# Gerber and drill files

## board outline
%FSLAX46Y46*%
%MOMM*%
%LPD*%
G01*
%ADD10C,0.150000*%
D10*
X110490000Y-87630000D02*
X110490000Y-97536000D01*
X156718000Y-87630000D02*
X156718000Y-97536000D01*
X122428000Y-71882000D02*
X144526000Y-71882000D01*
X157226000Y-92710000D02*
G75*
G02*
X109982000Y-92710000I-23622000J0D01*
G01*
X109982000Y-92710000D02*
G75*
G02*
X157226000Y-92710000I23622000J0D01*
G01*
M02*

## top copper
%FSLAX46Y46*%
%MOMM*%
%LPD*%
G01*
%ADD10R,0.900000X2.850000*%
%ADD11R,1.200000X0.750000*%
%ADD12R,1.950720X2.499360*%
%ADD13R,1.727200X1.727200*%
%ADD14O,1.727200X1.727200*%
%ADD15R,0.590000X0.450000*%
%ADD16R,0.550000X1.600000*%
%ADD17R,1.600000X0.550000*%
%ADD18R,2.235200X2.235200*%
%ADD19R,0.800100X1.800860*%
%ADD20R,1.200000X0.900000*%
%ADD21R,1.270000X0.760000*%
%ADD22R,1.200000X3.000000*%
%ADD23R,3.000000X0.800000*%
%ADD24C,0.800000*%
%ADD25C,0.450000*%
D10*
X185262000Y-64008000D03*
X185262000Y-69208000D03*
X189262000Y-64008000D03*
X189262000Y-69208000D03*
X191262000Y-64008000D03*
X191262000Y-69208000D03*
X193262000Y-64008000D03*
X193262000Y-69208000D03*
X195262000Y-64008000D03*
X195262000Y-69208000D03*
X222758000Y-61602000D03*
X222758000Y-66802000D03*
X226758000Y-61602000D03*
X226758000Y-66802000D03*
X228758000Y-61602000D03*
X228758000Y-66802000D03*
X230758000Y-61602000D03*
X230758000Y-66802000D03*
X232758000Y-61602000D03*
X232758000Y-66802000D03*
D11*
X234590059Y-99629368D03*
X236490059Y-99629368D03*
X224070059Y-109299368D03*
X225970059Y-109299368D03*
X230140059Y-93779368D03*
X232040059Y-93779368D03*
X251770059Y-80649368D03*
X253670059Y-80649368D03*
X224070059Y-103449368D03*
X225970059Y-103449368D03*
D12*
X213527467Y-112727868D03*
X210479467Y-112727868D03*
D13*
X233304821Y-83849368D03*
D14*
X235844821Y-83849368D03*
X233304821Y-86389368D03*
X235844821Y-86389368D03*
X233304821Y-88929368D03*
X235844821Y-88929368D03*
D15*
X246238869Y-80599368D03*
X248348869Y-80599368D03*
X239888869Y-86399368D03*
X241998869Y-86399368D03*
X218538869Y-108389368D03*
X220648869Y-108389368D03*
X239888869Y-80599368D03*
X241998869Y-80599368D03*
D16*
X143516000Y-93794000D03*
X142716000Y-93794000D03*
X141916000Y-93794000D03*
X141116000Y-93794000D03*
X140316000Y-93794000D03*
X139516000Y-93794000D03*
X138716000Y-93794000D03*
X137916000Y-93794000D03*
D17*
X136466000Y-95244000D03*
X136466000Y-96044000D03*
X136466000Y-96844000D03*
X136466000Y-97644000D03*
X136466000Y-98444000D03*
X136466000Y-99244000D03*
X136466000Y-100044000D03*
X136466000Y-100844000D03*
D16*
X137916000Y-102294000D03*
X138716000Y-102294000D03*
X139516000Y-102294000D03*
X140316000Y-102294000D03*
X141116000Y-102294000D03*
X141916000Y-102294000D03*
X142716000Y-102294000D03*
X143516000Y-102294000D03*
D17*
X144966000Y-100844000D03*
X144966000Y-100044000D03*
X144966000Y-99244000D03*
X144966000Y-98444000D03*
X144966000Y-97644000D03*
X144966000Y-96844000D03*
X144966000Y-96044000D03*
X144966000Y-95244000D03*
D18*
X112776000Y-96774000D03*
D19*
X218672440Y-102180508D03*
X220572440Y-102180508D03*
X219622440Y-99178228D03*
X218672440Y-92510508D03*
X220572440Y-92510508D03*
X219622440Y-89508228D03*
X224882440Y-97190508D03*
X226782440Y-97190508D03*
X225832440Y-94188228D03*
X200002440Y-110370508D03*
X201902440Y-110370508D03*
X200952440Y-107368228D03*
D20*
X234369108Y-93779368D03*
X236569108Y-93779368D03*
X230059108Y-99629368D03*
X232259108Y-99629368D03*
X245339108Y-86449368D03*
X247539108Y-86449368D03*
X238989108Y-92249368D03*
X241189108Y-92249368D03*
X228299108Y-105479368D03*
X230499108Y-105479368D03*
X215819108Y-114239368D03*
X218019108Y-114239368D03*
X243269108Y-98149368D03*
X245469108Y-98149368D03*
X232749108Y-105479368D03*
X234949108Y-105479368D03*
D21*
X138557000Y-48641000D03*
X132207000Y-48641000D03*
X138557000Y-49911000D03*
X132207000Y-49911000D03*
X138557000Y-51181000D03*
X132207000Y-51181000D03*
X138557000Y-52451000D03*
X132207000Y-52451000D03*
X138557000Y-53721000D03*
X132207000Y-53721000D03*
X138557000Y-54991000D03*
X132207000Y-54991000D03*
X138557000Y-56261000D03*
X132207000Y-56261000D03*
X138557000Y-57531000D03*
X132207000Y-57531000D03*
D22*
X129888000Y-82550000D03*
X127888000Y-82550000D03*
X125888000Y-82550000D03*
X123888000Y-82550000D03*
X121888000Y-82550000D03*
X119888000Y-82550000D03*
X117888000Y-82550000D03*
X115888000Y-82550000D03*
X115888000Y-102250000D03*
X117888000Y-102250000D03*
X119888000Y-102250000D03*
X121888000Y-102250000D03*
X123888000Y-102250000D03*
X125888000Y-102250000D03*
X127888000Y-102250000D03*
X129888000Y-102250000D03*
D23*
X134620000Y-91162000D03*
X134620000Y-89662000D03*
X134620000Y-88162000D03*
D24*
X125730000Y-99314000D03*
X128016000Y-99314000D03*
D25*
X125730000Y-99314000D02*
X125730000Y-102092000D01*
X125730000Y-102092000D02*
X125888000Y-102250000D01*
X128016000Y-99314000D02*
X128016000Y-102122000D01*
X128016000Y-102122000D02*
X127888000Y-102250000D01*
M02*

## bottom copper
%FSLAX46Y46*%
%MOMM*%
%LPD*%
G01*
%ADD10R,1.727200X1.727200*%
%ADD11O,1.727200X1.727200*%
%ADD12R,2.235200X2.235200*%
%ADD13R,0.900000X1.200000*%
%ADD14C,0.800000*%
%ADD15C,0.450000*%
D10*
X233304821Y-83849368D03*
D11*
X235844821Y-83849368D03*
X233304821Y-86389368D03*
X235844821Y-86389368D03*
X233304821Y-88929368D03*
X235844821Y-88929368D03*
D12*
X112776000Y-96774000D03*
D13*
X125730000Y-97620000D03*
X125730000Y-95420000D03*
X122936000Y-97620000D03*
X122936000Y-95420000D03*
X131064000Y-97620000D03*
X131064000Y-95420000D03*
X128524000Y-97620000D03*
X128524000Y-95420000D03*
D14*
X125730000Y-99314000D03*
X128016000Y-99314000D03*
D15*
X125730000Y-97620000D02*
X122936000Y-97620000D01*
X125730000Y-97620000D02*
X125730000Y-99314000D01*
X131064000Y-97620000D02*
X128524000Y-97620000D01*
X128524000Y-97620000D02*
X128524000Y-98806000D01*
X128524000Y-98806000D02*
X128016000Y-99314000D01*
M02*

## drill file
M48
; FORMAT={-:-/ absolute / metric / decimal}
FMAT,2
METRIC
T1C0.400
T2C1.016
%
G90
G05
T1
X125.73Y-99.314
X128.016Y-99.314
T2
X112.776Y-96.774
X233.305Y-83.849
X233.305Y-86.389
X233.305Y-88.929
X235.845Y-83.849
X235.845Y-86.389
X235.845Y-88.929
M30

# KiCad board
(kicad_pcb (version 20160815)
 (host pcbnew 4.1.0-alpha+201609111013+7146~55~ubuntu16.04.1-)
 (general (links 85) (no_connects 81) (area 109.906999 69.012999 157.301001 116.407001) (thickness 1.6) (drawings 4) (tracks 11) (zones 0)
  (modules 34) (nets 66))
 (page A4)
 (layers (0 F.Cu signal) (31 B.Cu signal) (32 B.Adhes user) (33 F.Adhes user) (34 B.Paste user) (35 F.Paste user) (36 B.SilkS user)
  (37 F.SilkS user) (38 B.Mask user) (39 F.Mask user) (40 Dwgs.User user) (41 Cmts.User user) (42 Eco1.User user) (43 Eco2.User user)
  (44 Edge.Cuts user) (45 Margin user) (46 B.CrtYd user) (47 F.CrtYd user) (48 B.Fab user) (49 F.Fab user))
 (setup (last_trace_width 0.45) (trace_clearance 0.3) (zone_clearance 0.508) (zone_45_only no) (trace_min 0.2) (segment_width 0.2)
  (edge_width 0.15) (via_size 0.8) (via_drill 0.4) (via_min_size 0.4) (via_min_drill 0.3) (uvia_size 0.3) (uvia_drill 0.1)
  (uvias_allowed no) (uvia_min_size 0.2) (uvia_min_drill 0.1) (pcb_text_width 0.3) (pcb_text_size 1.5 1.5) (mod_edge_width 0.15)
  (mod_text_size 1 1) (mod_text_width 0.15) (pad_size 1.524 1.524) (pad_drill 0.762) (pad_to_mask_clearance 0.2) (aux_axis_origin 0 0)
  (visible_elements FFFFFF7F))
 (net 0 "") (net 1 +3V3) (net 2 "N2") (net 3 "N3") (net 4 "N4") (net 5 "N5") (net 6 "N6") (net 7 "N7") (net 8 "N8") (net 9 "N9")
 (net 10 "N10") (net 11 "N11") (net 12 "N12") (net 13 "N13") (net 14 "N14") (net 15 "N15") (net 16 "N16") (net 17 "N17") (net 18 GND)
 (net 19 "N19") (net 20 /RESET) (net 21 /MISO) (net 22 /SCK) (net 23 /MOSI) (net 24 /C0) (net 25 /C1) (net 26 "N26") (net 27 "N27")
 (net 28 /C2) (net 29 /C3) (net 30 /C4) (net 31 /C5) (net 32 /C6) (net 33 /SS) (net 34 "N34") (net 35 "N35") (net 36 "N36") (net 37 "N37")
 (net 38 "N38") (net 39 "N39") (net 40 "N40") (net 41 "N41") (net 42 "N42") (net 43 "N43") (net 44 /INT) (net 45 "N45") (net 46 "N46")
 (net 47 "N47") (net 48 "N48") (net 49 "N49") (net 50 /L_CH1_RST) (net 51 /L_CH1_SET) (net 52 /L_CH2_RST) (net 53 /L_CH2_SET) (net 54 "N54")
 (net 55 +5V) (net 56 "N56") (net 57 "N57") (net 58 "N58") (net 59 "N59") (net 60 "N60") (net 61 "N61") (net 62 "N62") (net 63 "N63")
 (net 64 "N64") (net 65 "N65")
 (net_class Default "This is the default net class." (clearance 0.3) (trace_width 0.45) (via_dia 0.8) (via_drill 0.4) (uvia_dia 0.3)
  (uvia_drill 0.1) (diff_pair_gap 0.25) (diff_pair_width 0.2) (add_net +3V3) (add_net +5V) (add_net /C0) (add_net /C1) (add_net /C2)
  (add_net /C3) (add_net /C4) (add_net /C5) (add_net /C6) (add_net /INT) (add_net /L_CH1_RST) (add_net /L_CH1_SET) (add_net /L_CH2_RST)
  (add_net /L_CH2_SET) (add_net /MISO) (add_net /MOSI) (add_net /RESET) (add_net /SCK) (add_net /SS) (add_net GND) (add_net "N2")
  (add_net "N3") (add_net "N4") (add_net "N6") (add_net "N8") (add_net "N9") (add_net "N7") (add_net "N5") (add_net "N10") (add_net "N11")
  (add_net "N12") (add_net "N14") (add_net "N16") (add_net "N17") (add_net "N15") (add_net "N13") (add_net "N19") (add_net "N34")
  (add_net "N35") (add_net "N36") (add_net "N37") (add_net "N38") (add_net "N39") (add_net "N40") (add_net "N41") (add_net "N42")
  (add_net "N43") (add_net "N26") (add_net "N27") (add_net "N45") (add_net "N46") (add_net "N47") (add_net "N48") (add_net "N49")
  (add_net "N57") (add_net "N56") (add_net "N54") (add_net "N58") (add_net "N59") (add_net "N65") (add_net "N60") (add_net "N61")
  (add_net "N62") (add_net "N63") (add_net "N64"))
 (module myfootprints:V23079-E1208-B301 (layer F.Cu) (at 190.262 66.608)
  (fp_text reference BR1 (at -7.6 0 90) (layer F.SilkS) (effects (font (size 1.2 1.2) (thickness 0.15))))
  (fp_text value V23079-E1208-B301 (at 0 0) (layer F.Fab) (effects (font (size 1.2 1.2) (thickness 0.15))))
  (pad 12 smd rect (at -5 -2.6) (size 0.9 2.85) (layers F.Cu F.Paste F.Mask) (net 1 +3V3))
  (pad 1 smd rect (at -5 2.6) (size 0.9 2.85) (layers F.Cu F.Paste F.Mask) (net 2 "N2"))
  (pad 10 smd rect (at -1 -2.6) (size 0.9 2.85) (layers F.Cu F.Paste F.Mask) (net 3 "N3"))
  (pad 3 smd rect (at -1 2.6) (size 0.9 2.85) (layers F.Cu F.Paste F.Mask) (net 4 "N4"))
  (pad 9 smd rect (at 1 -2.6) (size 0.9 2.85) (layers F.Cu F.Paste F.Mask) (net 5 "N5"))
  (pad 4 smd rect (at 1 2.6) (size 0.9 2.85) (layers F.Cu F.Paste F.Mask) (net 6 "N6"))
  (pad 8 smd rect (at 3 -2.6) (size 0.9 2.85) (layers F.Cu F.Paste F.Mask) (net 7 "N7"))
  (pad 5 smd rect (at 3 2.6) (size 0.9 2.85) (layers F.Cu F.Paste F.Mask) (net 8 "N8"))
  (pad 7 smd rect (at 5 -2.6) (size 0.9 2.85) (layers F.Cu F.Paste F.Mask) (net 1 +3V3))
  (pad 6 smd rect (at 5 2.6) (size 0.9 2.85) (layers F.Cu F.Paste F.Mask) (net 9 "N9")))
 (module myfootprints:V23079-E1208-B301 (layer F.Cu) (at 227.758 64.202)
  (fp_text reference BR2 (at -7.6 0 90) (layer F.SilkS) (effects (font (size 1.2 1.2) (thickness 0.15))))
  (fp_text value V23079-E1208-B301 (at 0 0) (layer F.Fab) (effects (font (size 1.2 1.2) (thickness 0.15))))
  (pad 12 smd rect (at -5 -2.6) (size 0.9 2.85) (layers F.Cu F.Paste F.Mask) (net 1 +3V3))
  (pad 1 smd rect (at -5 2.6) (size 0.9 2.85) (layers F.Cu F.Paste F.Mask) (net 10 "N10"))
  (pad 10 smd rect (at -1 -2.6) (size 0.9 2.85) (layers F.Cu F.Paste F.Mask) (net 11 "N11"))
  (pad 3 smd rect (at -1 2.6) (size 0.9 2.85) (layers F.Cu F.Paste F.Mask) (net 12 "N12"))
  (pad 9 smd rect (at 1 -2.6) (size 0.9 2.85) (layers F.Cu F.Paste F.Mask) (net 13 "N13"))
  (pad 4 smd rect (at 1 2.6) (size 0.9 2.85) (layers F.Cu F.Paste F.Mask) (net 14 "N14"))
  (pad 8 smd rect (at 3 -2.6) (size 0.9 2.85) (layers F.Cu F.Paste F.Mask) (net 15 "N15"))
  (pad 5 smd rect (at 3 2.6) (size 0.9 2.85) (layers F.Cu F.Paste F.Mask) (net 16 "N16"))
  (pad 7 smd rect (at 5 -2.6) (size 0.9 2.85) (layers F.Cu F.Paste F.Mask) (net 1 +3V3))
  (pad 6 smd rect (at 5 2.6) (size 0.9 2.85) (layers F.Cu F.Paste F.Mask) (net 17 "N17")))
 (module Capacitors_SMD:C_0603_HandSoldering (layer F.Cu) (at 235.540059 99.629368)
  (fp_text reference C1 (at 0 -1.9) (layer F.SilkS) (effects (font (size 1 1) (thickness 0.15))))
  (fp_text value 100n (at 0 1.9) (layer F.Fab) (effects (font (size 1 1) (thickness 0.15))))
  (pad 1 smd rect (at -0.95 0) (size 1.2 0.75) (layers F.Cu F.Paste F.Mask) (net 1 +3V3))
  (pad 2 smd rect (at 0.95 0) (size 1.2 0.75) (layers F.Cu F.Paste F.Mask) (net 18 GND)))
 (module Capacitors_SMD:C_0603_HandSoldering (layer F.Cu) (at 225.020059 109.299368)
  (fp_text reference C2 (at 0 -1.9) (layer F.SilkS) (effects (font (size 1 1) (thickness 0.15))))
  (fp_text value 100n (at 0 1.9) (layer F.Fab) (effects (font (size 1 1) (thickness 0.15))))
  (pad 1 smd rect (at -0.95 0) (size 1.2 0.75) (layers F.Cu F.Paste F.Mask) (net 18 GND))
  (pad 2 smd rect (at 0.95 0) (size 1.2 0.75) (layers F.Cu F.Paste F.Mask) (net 1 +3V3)))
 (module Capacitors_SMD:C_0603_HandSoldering (layer F.Cu) (at 231.090059 93.779368)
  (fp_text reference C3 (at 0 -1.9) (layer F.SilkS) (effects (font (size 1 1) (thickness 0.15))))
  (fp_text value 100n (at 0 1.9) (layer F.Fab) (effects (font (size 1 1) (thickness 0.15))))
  (pad 1 smd rect (at -0.95 0) (size 1.2 0.75) (layers F.Cu F.Paste F.Mask) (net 18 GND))
  (pad 2 smd rect (at 0.95 0) (size 1.2 0.75) (layers F.Cu F.Paste F.Mask) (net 1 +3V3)))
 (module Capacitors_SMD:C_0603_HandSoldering (layer F.Cu) (at 252.720059 80.649368)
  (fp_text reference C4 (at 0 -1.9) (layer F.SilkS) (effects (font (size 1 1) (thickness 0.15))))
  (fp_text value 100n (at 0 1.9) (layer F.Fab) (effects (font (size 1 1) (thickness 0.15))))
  (pad 1 smd rect (at -0.95 0) (size 1.2 0.75) (layers F.Cu F.Paste F.Mask) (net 18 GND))
  (pad 2 smd rect (at 0.95 0) (size 1.2 0.75) (layers F.Cu F.Paste F.Mask) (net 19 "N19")))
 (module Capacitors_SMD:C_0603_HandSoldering (layer F.Cu) (at 225.020059 103.449368)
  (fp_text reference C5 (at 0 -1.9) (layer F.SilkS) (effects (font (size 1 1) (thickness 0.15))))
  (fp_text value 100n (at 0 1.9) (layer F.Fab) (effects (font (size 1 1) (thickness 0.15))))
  (pad 1 smd rect (at -0.95 0) (size 1.2 0.75) (layers F.Cu F.Paste F.Mask) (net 18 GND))
  (pad 2 smd rect (at 0.95 0) (size 1.2 0.75) (layers F.Cu F.Paste F.Mask) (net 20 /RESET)))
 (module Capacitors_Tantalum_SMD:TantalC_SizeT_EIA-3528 (layer F.Cu) (at 212.003467 112.727868)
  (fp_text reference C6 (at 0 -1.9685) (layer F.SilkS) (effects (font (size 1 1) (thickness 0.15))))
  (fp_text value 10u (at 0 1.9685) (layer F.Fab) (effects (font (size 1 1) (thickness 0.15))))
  (pad 1 smd rect (at 1.524 0) (size 1.95072 2.49936) (layers F.Cu F.Paste F.Mask) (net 1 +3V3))
  (pad 2 smd rect (at -1.524 0) (size 1.95072 2.49936) (layers F.Cu F.Paste F.Mask) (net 18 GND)))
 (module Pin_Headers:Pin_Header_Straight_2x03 (layer F.Cu) (at 233.304821 83.849368)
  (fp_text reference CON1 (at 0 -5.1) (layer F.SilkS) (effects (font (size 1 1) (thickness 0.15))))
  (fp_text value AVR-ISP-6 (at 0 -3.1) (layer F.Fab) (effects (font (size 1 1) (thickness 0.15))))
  (pad 1 thru_hole rect (at 0 0) (size 1.7272 1.7272) (drill 1.016) (layers *.Cu *.Mask F.SilkS) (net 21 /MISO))
  (pad 2 thru_hole oval (at 2.54 0) (size 1.7272 1.7272) (drill 1.016) (layers *.Cu *.Mask F.SilkS) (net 1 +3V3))
  (pad 3 thru_hole oval (at 0 2.54) (size 1.7272 1.7272) (drill 1.016) (layers *.Cu *.Mask F.SilkS) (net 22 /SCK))
  (pad 4 thru_hole oval (at 2.54 2.54) (size 1.7272 1.7272) (drill 1.016) (layers *.Cu *.Mask F.SilkS) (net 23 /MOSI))
  (pad 5 thru_hole oval (at 0 5.08) (size 1.7272 1.7272) (drill 1.016) (layers *.Cu *.Mask F.SilkS) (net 20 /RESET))
  (pad 6 thru_hole oval (at 2.54 5.08) (size 1.7272 1.7272) (drill 1.016) (layers *.Cu *.Mask F.SilkS) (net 18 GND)))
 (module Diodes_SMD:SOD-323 (layer F.Cu) (at 247.293869 80.599368)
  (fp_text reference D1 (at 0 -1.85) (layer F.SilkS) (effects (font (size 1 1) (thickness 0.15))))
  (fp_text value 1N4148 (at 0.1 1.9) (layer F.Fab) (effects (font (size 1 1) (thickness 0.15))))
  (pad 1 smd rect (at -1.055 0) (size 0.59 0.45) (layers F.Cu F.Paste F.Mask) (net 1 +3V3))
  (pad 2 smd rect (at 1.055 0) (size 0.59 0.45) (layers F.Cu F.Paste F.Mask) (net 2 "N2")))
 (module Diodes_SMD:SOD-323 (layer F.Cu) (at 240.943869 86.399368)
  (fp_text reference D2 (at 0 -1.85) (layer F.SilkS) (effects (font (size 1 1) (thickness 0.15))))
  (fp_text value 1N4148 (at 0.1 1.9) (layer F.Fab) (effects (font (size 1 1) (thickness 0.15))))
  (pad 1 smd rect (at -1.055 0) (size 0.59 0.45) (layers F.Cu F.Paste F.Mask) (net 1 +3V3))
  (pad 2 smd rect (at 1.055 0) (size 0.59 0.45) (layers F.Cu F.Paste F.Mask) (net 9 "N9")))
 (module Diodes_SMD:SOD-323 (layer F.Cu) (at 219.593869 108.389368)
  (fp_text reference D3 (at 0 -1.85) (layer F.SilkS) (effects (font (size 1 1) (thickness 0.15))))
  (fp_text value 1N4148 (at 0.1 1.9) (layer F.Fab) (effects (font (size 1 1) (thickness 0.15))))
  (pad 1 smd rect (at -1.055 0) (size 0.59 0.45) (layers F.Cu F.Paste F.Mask) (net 1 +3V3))
  (pad 2 smd rect (at 1.055 0) (size 0.59 0.45) (layers F.Cu F.Paste F.Mask) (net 10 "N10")))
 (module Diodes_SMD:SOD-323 (layer F.Cu) (at 240.943869 80.599368)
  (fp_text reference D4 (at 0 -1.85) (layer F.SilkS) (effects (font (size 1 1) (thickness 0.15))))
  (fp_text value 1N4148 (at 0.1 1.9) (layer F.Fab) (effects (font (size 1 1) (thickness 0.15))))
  (pad 1 smd rect (at -1.055 0) (size 0.59 0.45) (layers F.Cu F.Paste F.Mask) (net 1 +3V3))
  (pad 2 smd rect (at 1.055 0) (size 0.59 0.45) (layers F.Cu F.Paste F.Mask) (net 17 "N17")))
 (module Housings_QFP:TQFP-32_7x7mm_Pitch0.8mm (layer F.Cu) (at 140.716 98.044 270)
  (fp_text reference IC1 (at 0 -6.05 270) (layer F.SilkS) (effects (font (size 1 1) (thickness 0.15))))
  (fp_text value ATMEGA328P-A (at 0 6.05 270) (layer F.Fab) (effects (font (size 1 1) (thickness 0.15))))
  (pad 1 smd rect (at -4.25 -2.8 270) (size 1.6 0.55) (layers F.Cu F.Paste F.Mask) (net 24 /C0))
  (pad 2 smd rect (at -4.25 -2 270) (size 1.6 0.55) (layers F.Cu F.Paste F.Mask) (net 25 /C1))
  (pad 3 smd rect (at -4.25 -1.2 270) (size 1.6 0.55) (layers F.Cu F.Paste F.Mask) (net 18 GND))
  (pad 4 smd rect (at -4.25 -0.4 270) (size 1.6 0.55) (layers F.Cu F.Paste F.Mask) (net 1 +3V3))
  (pad 5 smd rect (at -4.25 0.4 270) (size 1.6 0.55) (layers F.Cu F.Paste F.Mask) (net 18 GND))
  (pad 6 smd rect (at -4.25 1.2 270) (size 1.6 0.55) (layers F.Cu F.Paste F.Mask) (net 1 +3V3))
  (pad 7 smd rect (at -4.25 2 270) (size 1.6 0.55) (layers F.Cu F.Paste F.Mask) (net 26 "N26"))
  (pad 8 smd rect (at -4.25 2.8 270) (size 1.6 0.55) (layers F.Cu F.Paste F.Mask) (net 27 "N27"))
  (pad 9 smd rect (at -2.8 4.25) (size 1.6 0.55) (layers F.Cu F.Paste F.Mask) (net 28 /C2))
  (pad 10 smd rect (at -2 4.25) (size 1.6 0.55) (layers F.Cu F.Paste F.Mask) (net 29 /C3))
  (pad 11 smd rect (at -1.2 4.25) (size 1.6 0.55) (layers F.Cu F.Paste F.Mask) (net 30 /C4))
  (pad 12 smd rect (at -0.4 4.25) (size 1.6 0.55) (layers F.Cu F.Paste F.Mask) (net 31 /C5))
  (pad 13 smd rect (at 0.4 4.25) (size 1.6 0.55) (layers F.Cu F.Paste F.Mask) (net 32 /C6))
  (pad 14 smd rect (at 1.2 4.25) (size 1.6 0.55) (layers F.Cu F.Paste F.Mask) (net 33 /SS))
  (pad 15 smd rect (at 2 4.25) (size 1.6 0.55) (layers F.Cu F.Paste F.Mask) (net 23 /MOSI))
  (pad 16 smd rect (at 2.8 4.25) (size 1.6 0.55) (layers F.Cu F.Paste F.Mask) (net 21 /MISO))
  (pad 17 smd rect (at 4.25 2.8 270) (size 1.6 0.55) (layers F.Cu F.Paste F.Mask) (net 22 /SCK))
  (pad 18 smd rect (at 4.25 2 270) (size 1.6 0.55) (layers F.Cu F.Paste F.Mask) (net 1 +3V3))
  (pad 19 smd rect (at 4.25 1.2 270) (size 1.6 0.55) (layers F.Cu F.Paste F.Mask) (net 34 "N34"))
  (pad 20 smd rect (at 4.25 0.4 270) (size 1.6 0.55) (layers F.Cu F.Paste F.Mask) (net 19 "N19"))
  (pad 21 smd rect (at 4.25 -0.4 270) (size 1.6 0.55) (layers F.Cu F.Paste F.Mask) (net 18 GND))
  (pad 22 smd rect (at 4.25 -1.2 270) (size 1.6 0.55) (layers F.Cu F.Paste F.Mask) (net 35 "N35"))
  (pad 23 smd rect (at 4.25 -2 270) (size 1.6 0.55) (layers F.Cu F.Paste F.Mask) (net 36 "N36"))
  (pad 24 smd rect (at 4.25 -2.8 270) (size 1.6 0.55) (layers F.Cu F.Paste F.Mask) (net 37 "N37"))
  (pad 25 smd rect (at 2.8 -4.25) (size 1.6 0.55) (layers F.Cu F.Paste F.Mask) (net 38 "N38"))
  (pad 26 smd rect (at 2 -4.25) (size 1.6 0.55) (layers F.Cu F.Paste F.Mask) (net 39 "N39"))
  (pad 27 smd rect (at 1.2 -4.25) (size 1.6 0.55) (layers F.Cu F.Paste F.Mask) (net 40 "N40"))
  (pad 28 smd rect (at 0.4 -4.25) (size 1.6 0.55) (layers F.Cu F.Paste F.Mask) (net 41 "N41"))
  (pad 29 smd rect (at -0.4 -4.25) (size 1.6 0.55) (layers F.Cu F.Paste F.Mask) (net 20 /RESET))
  (pad 30 smd rect (at -1.2 -4.25) (size 1.6 0.55) (layers F.Cu F.Paste F.Mask) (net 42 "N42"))
  (pad 31 smd rect (at -2 -4.25) (size 1.6 0.55) (layers F.Cu F.Paste F.Mask) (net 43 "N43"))
  (pad 32 smd rect (at -2.8 -4.25) (size 1.6 0.55) (layers F.Cu F.Paste F.Mask) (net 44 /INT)))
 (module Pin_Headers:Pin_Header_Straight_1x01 (layer F.Cu) (at 112.776 96.774)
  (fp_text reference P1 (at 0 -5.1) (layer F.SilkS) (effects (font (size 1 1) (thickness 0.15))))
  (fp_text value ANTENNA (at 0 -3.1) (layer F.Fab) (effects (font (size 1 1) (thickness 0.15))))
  (pad 1 thru_hole rect (at 0 0) (size 2.2352 2.2352) (drill 1.016) (layers *.Cu *.Mask F.SilkS) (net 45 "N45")))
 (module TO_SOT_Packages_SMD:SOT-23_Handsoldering (layer F.Cu) (at 219.62244 100.679368)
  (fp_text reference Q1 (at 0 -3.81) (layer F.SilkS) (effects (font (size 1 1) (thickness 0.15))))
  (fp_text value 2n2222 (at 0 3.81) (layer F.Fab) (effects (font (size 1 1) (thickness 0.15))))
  (pad 1 smd rect (at -0.95 1.50114) (size 0.8001 1.80086) (layers F.Cu F.Paste F.Mask) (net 2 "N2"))
  (pad 2 smd rect (at 0.95 1.50114) (size 0.8001 1.80086) (layers F.Cu F.Paste F.Mask) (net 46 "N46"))
  (pad 3 smd rect (at 0 -1.50114) (size 0.8001 1.80086) (layers F.Cu F.Paste F.Mask) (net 18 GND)))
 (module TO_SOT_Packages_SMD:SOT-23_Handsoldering (layer F.Cu) (at 219.62244 91.009368)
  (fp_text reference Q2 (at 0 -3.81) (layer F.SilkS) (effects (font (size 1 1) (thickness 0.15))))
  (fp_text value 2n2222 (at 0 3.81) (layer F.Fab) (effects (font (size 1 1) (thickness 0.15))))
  (pad 1 smd rect (at -0.95 1.50114) (size 0.8001 1.80086) (layers F.Cu F.Paste F.Mask) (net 9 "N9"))
  (pad 2 smd rect (at 0.95 1.50114) (size 0.8001 1.80086) (layers F.Cu F.Paste F.Mask) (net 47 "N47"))
  (pad 3 smd rect (at 0 -1.50114) (size 0.8001 1.80086) (layers F.Cu F.Paste F.Mask) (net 18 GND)))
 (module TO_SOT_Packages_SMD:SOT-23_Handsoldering (layer F.Cu) (at 225.83244 95.689368)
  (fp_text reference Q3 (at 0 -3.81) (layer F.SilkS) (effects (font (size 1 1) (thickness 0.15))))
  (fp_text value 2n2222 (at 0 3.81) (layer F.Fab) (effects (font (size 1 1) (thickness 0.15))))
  (pad 1 smd rect (at -0.95 1.50114) (size 0.8001 1.80086) (layers F.Cu F.Paste F.Mask) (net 10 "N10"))
  (pad 2 smd rect (at 0.95 1.50114) (size 0.8001 1.80086) (layers F.Cu F.Paste F.Mask) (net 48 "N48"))
  (pad 3 smd rect (at 0 -1.50114) (size 0.8001 1.80086) (layers F.Cu F.Paste F.Mask) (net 18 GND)))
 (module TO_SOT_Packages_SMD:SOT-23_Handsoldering (layer F.Cu) (at 200.95244 108.869368)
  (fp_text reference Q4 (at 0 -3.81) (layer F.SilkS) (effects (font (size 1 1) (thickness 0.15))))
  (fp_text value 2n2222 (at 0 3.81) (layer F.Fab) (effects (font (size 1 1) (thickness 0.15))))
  (pad 1 smd rect (at -0.95 1.50114) (size 0.8001 1.80086) (layers F.Cu F.Paste F.Mask) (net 17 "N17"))
  (pad 2 smd rect (at 0.95 1.50114) (size 0.8001 1.80086) (layers F.Cu F.Paste F.Mask) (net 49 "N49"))
  (pad 3 smd rect (at 0 -1.50114) (size 0.8001 1.80086) (layers F.Cu F.Paste F.Mask) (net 18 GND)))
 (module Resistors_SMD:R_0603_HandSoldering (layer F.Cu) (at 235.469108 93.779368)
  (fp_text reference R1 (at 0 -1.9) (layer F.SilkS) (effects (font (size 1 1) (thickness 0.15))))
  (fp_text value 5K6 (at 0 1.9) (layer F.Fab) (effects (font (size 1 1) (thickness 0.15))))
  (pad 1 smd rect (at -1.1 0) (size 1.2 0.9) (layers F.Cu F.Paste F.Mask) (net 46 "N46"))
  (pad 2 smd rect (at 1.1 0) (size 1.2 0.9) (layers F.Cu F.Paste F.Mask) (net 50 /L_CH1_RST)))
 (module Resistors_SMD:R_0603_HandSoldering (layer F.Cu) (at 231.159108 99.629368)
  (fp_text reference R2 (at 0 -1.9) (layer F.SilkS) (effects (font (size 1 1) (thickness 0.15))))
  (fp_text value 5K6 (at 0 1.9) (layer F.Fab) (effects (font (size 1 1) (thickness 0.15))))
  (pad 1 smd rect (at -1.1 0) (size 1.2 0.9) (layers F.Cu F.Paste F.Mask) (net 47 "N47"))
  (pad 2 smd rect (at 1.1 0) (size 1.2 0.9) (layers F.Cu F.Paste F.Mask) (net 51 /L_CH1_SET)))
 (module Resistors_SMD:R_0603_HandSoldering (layer F.Cu) (at 246.439108 86.449368)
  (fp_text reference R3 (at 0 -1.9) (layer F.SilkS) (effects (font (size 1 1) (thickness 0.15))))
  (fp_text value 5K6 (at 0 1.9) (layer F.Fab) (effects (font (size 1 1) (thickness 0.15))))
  (pad 1 smd rect (at -1.1 0) (size 1.2 0.9) (layers F.Cu F.Paste F.Mask) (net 48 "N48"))
  (pad 2 smd rect (at 1.1 0) (size 1.2 0.9) (layers F.Cu F.Paste F.Mask) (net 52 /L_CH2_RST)))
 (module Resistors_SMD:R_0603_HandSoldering (layer F.Cu) (at 240.089108 92.249368)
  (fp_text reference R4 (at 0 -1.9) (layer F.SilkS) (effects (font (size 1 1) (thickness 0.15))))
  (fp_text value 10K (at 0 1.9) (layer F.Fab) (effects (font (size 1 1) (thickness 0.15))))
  (pad 1 smd rect (at -1.1 0) (size 1.2 0.9) (layers F.Cu F.Paste F.Mask) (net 1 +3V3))
  (pad 2 smd rect (at 1.1 0) (size 1.2 0.9) (layers F.Cu F.Paste F.Mask) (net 20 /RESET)))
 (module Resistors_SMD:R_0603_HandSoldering (layer F.Cu) (at 229.399108 105.479368)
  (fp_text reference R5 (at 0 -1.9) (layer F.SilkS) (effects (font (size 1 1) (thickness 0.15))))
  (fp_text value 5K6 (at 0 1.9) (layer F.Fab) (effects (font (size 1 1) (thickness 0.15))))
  (pad 1 smd rect (at -1.1 0) (size 1.2 0.9) (layers F.Cu F.Paste F.Mask) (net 49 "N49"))
  (pad 2 smd rect (at 1.1 0) (size 1.2 0.9) (layers F.Cu F.Paste F.Mask) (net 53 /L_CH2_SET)))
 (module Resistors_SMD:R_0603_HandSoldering (layer B.Cu) (at 125.73 96.52 90)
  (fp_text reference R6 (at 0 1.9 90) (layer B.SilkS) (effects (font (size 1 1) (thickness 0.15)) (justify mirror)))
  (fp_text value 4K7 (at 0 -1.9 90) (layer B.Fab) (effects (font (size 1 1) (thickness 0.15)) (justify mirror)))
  (pad 1 smd rect (at -1.1 0 90) (size 1.2 0.9) (layers B.Cu B.Paste B.Mask) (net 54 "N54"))
  (pad 2 smd rect (at 1.1 0 90) (size 1.2 0.9) (layers B.Cu B.Paste B.Mask) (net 23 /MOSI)))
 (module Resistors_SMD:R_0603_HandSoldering (layer B.Cu) (at 122.936 96.52 90)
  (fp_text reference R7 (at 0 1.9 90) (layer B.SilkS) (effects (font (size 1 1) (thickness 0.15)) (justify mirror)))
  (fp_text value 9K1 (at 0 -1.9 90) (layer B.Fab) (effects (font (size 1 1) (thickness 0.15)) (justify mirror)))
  (pad 1 smd rect (at -1.1 0 90) (size 1.2 0.9) (layers B.Cu B.Paste B.Mask) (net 54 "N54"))
  (pad 2 smd rect (at 1.1 0 90) (size 1.2 0.9) (layers B.Cu B.Paste B.Mask) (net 18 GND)))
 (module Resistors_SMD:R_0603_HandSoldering (layer F.Cu) (at 216.919108 114.239368)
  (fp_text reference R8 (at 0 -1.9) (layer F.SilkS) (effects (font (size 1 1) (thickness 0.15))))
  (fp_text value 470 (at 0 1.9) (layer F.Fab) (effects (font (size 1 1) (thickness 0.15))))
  (pad 1 smd rect (at -1.1 0) (size 1.2 0.9) (layers F.Cu F.Paste F.Mask) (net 33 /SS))
  (pad 2 smd rect (at 1.1 0) (size 1.2 0.9) (layers F.Cu F.Paste F.Mask) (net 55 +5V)))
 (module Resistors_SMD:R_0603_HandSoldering (layer B.Cu) (at 131.064 96.52 90)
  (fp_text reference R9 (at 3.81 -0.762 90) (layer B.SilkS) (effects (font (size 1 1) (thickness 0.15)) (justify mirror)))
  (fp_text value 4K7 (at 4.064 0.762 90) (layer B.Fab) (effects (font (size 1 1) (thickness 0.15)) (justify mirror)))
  (pad 1 smd rect (at -1.1 0 90) (size 1.2 0.9) (layers B.Cu B.Paste B.Mask) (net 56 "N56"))
  (pad 2 smd rect (at 1.1 0 90) (size 1.2 0.9) (layers B.Cu B.Paste B.Mask) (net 33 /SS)))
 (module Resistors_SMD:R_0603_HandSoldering (layer F.Cu) (at 244.369108 98.149368)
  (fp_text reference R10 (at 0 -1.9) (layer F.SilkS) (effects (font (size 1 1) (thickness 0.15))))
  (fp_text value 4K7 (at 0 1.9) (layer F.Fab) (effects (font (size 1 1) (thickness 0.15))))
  (pad 1 smd rect (at -1.1 0) (size 1.2 0.9) (layers F.Cu F.Paste F.Mask) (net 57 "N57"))
  (pad 2 smd rect (at 1.1 0) (size 1.2 0.9) (layers F.Cu F.Paste F.Mask) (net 22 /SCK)))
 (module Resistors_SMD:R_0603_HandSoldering (layer B.Cu) (at 128.524 96.52 90)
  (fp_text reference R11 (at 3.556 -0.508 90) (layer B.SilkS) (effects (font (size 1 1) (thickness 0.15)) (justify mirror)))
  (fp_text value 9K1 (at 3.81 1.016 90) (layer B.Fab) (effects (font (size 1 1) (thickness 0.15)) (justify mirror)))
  (pad 1 smd rect (at -1.1 0 90) (size 1.2 0.9) (layers B.Cu B.Paste B.Mask) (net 56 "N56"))
  (pad 2 smd rect (at 1.1 0 90) (size 1.2 0.9) (layers B.Cu B.Paste B.Mask) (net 18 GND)))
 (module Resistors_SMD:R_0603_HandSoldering (layer F.Cu) (at 233.849108 105.479368)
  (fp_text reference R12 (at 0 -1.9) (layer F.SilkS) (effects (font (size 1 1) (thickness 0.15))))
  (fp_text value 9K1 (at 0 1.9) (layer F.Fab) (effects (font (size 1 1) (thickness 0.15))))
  (pad 1 smd rect (at -1.1 0) (size 1.2 0.9) (layers F.Cu F.Paste F.Mask) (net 57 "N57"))
  (pad 2 smd rect (at 1.1 0) (size 1.2 0.9) (layers F.Cu F.Paste F.Mask) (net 18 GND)))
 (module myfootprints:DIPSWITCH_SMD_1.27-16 (layer F.Cu) (at 135.382 53.086 270)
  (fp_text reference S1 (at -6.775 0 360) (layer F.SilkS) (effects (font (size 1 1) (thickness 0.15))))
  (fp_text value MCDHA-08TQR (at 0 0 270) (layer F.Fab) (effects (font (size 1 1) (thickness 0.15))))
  (pad 16 smd rect (at -4.445 -3.175 270) (size 0.76 1.27) (layers F.Cu F.Paste F.Mask) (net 18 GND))
  (pad 1 smd rect (at -4.445 3.175 270) (size 0.76 1.27) (layers F.Cu F.Paste F.Mask) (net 24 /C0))
  (pad 15 smd rect (at -3.175 -3.175 270) (size 0.76 1.27) (layers F.Cu F.Paste F.Mask) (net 18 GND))
  (pad 2 smd rect (at -3.175 3.175 270) (size 0.76 1.27) (layers F.Cu F.Paste F.Mask) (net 25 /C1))
  (pad 14 smd rect (at -1.905 -3.175 270) (size 0.76 1.27) (layers F.Cu F.Paste F.Mask) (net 18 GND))
  (pad 3 smd rect (at -1.905 3.175 270) (size 0.76 1.27) (layers F.Cu F.Paste F.Mask) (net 28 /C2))
  (pad 13 smd rect (at -0.635 -3.175 270) (size 0.76 1.27) (layers F.Cu F.Paste F.Mask) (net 18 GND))
  (pad 4 smd rect (at -0.635 3.175 270) (size 0.76 1.27) (layers F.Cu F.Paste F.Mask) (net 29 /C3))
  (pad 12 smd rect (at 0.635 -3.175 270) (size 0.76 1.27) (layers F.Cu F.Paste F.Mask) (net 18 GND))
  (pad 5 smd rect (at 0.635 3.175 270) (size 0.76 1.27) (layers F.Cu F.Paste F.Mask) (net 30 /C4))
  (pad 11 smd rect (at 1.905 -3.175 270) (size 0.76 1.27) (layers F.Cu F.Paste F.Mask) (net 18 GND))
  (pad 6 smd rect (at 1.905 3.175 270) (size 0.76 1.27) (layers F.Cu F.Paste F.Mask) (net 31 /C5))
  (pad 10 smd rect (at 3.175 -3.175 270) (size 0.76 1.27) (layers F.Cu F.Paste F.Mask) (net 18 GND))
  (pad 7 smd rect (at 3.175 3.175 270) (size 0.76 1.27) (layers F.Cu F.Paste F.Mask) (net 32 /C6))
  (pad 9 smd rect (at 4.445 -3.175 270) (size 0.76 1.27) (layers F.Cu F.Paste F.Mask) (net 18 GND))
  (pad 8 smd rect (at 4.445 3.175 270) (size 0.76 1.27) (layers F.Cu F.Paste F.Mask) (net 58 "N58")))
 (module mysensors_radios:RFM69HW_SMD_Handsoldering (layer F.Cu) (at 129.888 83.95 270)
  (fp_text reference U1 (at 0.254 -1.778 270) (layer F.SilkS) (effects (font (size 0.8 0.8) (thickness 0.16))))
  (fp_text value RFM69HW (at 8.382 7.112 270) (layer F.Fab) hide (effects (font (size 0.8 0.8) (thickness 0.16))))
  (pad 1 smd rect (at -1.4 0 270) (size 3 1.2) (layers F.Cu F.Paste F.Mask) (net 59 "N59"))
  (pad 2 smd rect (at -1.4 2 270) (size 3 1.2) (layers F.Cu F.Paste F.Mask) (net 44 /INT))
  (pad 3 smd rect (at -1.4 4 270) (size 3 1.2) (layers F.Cu F.Paste F.Mask) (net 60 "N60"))
  (pad 4 smd rect (at -1.4 6 270) (size 3 1.2) (layers F.Cu F.Paste F.Mask) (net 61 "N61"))
  (pad 5 smd rect (at -1.4 8 270) (size 3 1.2) (layers F.Cu F.Paste F.Mask) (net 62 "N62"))
  (pad 6 smd rect (at -1.4 10 270) (size 3 1.2) (layers F.Cu F.Paste F.Mask) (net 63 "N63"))
  (pad 7 smd rect (at -1.4 12 270) (size 3 1.2) (layers F.Cu F.Paste F.Mask) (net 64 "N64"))
  (pad 8 smd rect (at -1.4 14 270) (size 3 1.2) (layers F.Cu F.Paste F.Mask) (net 1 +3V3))
  (pad 9 smd rect (at 18.3 14 270) (size 3 1.2) (layers F.Cu F.Paste F.Mask) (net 18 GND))
  (pad 10 smd rect (at 18.3 12 270) (size 3 1.2) (layers F.Cu F.Paste F.Mask) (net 45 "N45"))
  (pad 11 smd rect (at 18.3 10 270) (size 3 1.2) (layers F.Cu F.Paste F.Mask) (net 18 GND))
  (pad 12 smd rect (at 18.3 8 270) (size 3 1.2) (layers F.Cu F.Paste F.Mask) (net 57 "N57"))
  (pad 13 smd rect (at 18.3 6 270) (size 3 1.2) (layers F.Cu F.Paste F.Mask) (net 21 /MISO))
  (pad 14 smd rect (at 18.3 4 270) (size 3 1.2) (layers F.Cu F.Paste F.Mask) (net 54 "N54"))
  (pad 15 smd rect (at 18.3 2 270) (size 3 1.2) (layers F.Cu F.Paste F.Mask) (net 56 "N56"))
  (pad 16 smd rect (at 18.3 0 270) (size 3 1.2) (layers F.Cu F.Paste F.Mask) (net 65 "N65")))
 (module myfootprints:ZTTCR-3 (layer F.Cu) (at 134.62 89.662 90)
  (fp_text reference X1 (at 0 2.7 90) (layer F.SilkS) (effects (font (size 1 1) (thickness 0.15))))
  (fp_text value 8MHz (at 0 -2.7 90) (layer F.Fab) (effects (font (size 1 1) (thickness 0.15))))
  (pad 1 smd rect (at -1.5 0 90) (size 0.8 3) (layers F.Cu F.Paste F.Mask) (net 27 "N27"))
  (pad 2 smd rect (at 0 0 90) (size 0.8 3) (layers F.Cu F.Paste F.Mask) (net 26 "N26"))
  (pad 3 smd rect (at 1.5 0 90) (size 0.8 3) (layers F.Cu F.Paste F.Mask) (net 18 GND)))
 (gr_line (start 110.49 87.63) (end 110.49 97.536) (layer Edge.Cuts) (width 0.15))
 (gr_line (start 156.718 87.63) (end 156.718 97.536) (layer Edge.Cuts) (width 0.15))
 (gr_line (start 122.428 71.882) (end 144.526 71.882) (layer Edge.Cuts) (width 0.15))
 (gr_circle (center 133.604 92.71) (end 157.226 92.71) (layer Edge.Cuts) (width 0.15))
 (segment (start 125.73 97.62) (end 122.936 97.62) (width 0.45) (layer B.Cu) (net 54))
 (segment (start 125.73 99.314) (end 125.73 102.092) (width 0.45) (layer F.Cu) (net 54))
 (segment (start 125.73 102.092) (end 125.888 102.25) (width 0.45) (layer F.Cu) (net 54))
 (segment (start 125.73 97.62) (end 125.73 99.314) (width 0.45) (layer B.Cu) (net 54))
 (via (at 125.73 99.314) (size 0.8) (drill 0.4) (layers F.Cu B.Cu) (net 54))
 (segment (start 131.064 97.62) (end 128.524 97.62) (width 0.45) (layer B.Cu) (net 56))
 (segment (start 128.016 99.314) (end 128.016 102.122) (width 0.45) (layer F.Cu) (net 56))
 (segment (start 128.016 102.122) (end 127.888 102.25) (width 0.45) (layer F.Cu) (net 56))
 (segment (start 128.524 97.62) (end 128.524 98.806) (width 0.45) (layer B.Cu) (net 56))
 (segment (start 128.524 98.806) (end 128.016 99.314) (width 0.45) (layer B.Cu) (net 56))
 (via (at 128.016 99.314) (size 0.8) (drill 0.4) (layers F.Cu B.Cu) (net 56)))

